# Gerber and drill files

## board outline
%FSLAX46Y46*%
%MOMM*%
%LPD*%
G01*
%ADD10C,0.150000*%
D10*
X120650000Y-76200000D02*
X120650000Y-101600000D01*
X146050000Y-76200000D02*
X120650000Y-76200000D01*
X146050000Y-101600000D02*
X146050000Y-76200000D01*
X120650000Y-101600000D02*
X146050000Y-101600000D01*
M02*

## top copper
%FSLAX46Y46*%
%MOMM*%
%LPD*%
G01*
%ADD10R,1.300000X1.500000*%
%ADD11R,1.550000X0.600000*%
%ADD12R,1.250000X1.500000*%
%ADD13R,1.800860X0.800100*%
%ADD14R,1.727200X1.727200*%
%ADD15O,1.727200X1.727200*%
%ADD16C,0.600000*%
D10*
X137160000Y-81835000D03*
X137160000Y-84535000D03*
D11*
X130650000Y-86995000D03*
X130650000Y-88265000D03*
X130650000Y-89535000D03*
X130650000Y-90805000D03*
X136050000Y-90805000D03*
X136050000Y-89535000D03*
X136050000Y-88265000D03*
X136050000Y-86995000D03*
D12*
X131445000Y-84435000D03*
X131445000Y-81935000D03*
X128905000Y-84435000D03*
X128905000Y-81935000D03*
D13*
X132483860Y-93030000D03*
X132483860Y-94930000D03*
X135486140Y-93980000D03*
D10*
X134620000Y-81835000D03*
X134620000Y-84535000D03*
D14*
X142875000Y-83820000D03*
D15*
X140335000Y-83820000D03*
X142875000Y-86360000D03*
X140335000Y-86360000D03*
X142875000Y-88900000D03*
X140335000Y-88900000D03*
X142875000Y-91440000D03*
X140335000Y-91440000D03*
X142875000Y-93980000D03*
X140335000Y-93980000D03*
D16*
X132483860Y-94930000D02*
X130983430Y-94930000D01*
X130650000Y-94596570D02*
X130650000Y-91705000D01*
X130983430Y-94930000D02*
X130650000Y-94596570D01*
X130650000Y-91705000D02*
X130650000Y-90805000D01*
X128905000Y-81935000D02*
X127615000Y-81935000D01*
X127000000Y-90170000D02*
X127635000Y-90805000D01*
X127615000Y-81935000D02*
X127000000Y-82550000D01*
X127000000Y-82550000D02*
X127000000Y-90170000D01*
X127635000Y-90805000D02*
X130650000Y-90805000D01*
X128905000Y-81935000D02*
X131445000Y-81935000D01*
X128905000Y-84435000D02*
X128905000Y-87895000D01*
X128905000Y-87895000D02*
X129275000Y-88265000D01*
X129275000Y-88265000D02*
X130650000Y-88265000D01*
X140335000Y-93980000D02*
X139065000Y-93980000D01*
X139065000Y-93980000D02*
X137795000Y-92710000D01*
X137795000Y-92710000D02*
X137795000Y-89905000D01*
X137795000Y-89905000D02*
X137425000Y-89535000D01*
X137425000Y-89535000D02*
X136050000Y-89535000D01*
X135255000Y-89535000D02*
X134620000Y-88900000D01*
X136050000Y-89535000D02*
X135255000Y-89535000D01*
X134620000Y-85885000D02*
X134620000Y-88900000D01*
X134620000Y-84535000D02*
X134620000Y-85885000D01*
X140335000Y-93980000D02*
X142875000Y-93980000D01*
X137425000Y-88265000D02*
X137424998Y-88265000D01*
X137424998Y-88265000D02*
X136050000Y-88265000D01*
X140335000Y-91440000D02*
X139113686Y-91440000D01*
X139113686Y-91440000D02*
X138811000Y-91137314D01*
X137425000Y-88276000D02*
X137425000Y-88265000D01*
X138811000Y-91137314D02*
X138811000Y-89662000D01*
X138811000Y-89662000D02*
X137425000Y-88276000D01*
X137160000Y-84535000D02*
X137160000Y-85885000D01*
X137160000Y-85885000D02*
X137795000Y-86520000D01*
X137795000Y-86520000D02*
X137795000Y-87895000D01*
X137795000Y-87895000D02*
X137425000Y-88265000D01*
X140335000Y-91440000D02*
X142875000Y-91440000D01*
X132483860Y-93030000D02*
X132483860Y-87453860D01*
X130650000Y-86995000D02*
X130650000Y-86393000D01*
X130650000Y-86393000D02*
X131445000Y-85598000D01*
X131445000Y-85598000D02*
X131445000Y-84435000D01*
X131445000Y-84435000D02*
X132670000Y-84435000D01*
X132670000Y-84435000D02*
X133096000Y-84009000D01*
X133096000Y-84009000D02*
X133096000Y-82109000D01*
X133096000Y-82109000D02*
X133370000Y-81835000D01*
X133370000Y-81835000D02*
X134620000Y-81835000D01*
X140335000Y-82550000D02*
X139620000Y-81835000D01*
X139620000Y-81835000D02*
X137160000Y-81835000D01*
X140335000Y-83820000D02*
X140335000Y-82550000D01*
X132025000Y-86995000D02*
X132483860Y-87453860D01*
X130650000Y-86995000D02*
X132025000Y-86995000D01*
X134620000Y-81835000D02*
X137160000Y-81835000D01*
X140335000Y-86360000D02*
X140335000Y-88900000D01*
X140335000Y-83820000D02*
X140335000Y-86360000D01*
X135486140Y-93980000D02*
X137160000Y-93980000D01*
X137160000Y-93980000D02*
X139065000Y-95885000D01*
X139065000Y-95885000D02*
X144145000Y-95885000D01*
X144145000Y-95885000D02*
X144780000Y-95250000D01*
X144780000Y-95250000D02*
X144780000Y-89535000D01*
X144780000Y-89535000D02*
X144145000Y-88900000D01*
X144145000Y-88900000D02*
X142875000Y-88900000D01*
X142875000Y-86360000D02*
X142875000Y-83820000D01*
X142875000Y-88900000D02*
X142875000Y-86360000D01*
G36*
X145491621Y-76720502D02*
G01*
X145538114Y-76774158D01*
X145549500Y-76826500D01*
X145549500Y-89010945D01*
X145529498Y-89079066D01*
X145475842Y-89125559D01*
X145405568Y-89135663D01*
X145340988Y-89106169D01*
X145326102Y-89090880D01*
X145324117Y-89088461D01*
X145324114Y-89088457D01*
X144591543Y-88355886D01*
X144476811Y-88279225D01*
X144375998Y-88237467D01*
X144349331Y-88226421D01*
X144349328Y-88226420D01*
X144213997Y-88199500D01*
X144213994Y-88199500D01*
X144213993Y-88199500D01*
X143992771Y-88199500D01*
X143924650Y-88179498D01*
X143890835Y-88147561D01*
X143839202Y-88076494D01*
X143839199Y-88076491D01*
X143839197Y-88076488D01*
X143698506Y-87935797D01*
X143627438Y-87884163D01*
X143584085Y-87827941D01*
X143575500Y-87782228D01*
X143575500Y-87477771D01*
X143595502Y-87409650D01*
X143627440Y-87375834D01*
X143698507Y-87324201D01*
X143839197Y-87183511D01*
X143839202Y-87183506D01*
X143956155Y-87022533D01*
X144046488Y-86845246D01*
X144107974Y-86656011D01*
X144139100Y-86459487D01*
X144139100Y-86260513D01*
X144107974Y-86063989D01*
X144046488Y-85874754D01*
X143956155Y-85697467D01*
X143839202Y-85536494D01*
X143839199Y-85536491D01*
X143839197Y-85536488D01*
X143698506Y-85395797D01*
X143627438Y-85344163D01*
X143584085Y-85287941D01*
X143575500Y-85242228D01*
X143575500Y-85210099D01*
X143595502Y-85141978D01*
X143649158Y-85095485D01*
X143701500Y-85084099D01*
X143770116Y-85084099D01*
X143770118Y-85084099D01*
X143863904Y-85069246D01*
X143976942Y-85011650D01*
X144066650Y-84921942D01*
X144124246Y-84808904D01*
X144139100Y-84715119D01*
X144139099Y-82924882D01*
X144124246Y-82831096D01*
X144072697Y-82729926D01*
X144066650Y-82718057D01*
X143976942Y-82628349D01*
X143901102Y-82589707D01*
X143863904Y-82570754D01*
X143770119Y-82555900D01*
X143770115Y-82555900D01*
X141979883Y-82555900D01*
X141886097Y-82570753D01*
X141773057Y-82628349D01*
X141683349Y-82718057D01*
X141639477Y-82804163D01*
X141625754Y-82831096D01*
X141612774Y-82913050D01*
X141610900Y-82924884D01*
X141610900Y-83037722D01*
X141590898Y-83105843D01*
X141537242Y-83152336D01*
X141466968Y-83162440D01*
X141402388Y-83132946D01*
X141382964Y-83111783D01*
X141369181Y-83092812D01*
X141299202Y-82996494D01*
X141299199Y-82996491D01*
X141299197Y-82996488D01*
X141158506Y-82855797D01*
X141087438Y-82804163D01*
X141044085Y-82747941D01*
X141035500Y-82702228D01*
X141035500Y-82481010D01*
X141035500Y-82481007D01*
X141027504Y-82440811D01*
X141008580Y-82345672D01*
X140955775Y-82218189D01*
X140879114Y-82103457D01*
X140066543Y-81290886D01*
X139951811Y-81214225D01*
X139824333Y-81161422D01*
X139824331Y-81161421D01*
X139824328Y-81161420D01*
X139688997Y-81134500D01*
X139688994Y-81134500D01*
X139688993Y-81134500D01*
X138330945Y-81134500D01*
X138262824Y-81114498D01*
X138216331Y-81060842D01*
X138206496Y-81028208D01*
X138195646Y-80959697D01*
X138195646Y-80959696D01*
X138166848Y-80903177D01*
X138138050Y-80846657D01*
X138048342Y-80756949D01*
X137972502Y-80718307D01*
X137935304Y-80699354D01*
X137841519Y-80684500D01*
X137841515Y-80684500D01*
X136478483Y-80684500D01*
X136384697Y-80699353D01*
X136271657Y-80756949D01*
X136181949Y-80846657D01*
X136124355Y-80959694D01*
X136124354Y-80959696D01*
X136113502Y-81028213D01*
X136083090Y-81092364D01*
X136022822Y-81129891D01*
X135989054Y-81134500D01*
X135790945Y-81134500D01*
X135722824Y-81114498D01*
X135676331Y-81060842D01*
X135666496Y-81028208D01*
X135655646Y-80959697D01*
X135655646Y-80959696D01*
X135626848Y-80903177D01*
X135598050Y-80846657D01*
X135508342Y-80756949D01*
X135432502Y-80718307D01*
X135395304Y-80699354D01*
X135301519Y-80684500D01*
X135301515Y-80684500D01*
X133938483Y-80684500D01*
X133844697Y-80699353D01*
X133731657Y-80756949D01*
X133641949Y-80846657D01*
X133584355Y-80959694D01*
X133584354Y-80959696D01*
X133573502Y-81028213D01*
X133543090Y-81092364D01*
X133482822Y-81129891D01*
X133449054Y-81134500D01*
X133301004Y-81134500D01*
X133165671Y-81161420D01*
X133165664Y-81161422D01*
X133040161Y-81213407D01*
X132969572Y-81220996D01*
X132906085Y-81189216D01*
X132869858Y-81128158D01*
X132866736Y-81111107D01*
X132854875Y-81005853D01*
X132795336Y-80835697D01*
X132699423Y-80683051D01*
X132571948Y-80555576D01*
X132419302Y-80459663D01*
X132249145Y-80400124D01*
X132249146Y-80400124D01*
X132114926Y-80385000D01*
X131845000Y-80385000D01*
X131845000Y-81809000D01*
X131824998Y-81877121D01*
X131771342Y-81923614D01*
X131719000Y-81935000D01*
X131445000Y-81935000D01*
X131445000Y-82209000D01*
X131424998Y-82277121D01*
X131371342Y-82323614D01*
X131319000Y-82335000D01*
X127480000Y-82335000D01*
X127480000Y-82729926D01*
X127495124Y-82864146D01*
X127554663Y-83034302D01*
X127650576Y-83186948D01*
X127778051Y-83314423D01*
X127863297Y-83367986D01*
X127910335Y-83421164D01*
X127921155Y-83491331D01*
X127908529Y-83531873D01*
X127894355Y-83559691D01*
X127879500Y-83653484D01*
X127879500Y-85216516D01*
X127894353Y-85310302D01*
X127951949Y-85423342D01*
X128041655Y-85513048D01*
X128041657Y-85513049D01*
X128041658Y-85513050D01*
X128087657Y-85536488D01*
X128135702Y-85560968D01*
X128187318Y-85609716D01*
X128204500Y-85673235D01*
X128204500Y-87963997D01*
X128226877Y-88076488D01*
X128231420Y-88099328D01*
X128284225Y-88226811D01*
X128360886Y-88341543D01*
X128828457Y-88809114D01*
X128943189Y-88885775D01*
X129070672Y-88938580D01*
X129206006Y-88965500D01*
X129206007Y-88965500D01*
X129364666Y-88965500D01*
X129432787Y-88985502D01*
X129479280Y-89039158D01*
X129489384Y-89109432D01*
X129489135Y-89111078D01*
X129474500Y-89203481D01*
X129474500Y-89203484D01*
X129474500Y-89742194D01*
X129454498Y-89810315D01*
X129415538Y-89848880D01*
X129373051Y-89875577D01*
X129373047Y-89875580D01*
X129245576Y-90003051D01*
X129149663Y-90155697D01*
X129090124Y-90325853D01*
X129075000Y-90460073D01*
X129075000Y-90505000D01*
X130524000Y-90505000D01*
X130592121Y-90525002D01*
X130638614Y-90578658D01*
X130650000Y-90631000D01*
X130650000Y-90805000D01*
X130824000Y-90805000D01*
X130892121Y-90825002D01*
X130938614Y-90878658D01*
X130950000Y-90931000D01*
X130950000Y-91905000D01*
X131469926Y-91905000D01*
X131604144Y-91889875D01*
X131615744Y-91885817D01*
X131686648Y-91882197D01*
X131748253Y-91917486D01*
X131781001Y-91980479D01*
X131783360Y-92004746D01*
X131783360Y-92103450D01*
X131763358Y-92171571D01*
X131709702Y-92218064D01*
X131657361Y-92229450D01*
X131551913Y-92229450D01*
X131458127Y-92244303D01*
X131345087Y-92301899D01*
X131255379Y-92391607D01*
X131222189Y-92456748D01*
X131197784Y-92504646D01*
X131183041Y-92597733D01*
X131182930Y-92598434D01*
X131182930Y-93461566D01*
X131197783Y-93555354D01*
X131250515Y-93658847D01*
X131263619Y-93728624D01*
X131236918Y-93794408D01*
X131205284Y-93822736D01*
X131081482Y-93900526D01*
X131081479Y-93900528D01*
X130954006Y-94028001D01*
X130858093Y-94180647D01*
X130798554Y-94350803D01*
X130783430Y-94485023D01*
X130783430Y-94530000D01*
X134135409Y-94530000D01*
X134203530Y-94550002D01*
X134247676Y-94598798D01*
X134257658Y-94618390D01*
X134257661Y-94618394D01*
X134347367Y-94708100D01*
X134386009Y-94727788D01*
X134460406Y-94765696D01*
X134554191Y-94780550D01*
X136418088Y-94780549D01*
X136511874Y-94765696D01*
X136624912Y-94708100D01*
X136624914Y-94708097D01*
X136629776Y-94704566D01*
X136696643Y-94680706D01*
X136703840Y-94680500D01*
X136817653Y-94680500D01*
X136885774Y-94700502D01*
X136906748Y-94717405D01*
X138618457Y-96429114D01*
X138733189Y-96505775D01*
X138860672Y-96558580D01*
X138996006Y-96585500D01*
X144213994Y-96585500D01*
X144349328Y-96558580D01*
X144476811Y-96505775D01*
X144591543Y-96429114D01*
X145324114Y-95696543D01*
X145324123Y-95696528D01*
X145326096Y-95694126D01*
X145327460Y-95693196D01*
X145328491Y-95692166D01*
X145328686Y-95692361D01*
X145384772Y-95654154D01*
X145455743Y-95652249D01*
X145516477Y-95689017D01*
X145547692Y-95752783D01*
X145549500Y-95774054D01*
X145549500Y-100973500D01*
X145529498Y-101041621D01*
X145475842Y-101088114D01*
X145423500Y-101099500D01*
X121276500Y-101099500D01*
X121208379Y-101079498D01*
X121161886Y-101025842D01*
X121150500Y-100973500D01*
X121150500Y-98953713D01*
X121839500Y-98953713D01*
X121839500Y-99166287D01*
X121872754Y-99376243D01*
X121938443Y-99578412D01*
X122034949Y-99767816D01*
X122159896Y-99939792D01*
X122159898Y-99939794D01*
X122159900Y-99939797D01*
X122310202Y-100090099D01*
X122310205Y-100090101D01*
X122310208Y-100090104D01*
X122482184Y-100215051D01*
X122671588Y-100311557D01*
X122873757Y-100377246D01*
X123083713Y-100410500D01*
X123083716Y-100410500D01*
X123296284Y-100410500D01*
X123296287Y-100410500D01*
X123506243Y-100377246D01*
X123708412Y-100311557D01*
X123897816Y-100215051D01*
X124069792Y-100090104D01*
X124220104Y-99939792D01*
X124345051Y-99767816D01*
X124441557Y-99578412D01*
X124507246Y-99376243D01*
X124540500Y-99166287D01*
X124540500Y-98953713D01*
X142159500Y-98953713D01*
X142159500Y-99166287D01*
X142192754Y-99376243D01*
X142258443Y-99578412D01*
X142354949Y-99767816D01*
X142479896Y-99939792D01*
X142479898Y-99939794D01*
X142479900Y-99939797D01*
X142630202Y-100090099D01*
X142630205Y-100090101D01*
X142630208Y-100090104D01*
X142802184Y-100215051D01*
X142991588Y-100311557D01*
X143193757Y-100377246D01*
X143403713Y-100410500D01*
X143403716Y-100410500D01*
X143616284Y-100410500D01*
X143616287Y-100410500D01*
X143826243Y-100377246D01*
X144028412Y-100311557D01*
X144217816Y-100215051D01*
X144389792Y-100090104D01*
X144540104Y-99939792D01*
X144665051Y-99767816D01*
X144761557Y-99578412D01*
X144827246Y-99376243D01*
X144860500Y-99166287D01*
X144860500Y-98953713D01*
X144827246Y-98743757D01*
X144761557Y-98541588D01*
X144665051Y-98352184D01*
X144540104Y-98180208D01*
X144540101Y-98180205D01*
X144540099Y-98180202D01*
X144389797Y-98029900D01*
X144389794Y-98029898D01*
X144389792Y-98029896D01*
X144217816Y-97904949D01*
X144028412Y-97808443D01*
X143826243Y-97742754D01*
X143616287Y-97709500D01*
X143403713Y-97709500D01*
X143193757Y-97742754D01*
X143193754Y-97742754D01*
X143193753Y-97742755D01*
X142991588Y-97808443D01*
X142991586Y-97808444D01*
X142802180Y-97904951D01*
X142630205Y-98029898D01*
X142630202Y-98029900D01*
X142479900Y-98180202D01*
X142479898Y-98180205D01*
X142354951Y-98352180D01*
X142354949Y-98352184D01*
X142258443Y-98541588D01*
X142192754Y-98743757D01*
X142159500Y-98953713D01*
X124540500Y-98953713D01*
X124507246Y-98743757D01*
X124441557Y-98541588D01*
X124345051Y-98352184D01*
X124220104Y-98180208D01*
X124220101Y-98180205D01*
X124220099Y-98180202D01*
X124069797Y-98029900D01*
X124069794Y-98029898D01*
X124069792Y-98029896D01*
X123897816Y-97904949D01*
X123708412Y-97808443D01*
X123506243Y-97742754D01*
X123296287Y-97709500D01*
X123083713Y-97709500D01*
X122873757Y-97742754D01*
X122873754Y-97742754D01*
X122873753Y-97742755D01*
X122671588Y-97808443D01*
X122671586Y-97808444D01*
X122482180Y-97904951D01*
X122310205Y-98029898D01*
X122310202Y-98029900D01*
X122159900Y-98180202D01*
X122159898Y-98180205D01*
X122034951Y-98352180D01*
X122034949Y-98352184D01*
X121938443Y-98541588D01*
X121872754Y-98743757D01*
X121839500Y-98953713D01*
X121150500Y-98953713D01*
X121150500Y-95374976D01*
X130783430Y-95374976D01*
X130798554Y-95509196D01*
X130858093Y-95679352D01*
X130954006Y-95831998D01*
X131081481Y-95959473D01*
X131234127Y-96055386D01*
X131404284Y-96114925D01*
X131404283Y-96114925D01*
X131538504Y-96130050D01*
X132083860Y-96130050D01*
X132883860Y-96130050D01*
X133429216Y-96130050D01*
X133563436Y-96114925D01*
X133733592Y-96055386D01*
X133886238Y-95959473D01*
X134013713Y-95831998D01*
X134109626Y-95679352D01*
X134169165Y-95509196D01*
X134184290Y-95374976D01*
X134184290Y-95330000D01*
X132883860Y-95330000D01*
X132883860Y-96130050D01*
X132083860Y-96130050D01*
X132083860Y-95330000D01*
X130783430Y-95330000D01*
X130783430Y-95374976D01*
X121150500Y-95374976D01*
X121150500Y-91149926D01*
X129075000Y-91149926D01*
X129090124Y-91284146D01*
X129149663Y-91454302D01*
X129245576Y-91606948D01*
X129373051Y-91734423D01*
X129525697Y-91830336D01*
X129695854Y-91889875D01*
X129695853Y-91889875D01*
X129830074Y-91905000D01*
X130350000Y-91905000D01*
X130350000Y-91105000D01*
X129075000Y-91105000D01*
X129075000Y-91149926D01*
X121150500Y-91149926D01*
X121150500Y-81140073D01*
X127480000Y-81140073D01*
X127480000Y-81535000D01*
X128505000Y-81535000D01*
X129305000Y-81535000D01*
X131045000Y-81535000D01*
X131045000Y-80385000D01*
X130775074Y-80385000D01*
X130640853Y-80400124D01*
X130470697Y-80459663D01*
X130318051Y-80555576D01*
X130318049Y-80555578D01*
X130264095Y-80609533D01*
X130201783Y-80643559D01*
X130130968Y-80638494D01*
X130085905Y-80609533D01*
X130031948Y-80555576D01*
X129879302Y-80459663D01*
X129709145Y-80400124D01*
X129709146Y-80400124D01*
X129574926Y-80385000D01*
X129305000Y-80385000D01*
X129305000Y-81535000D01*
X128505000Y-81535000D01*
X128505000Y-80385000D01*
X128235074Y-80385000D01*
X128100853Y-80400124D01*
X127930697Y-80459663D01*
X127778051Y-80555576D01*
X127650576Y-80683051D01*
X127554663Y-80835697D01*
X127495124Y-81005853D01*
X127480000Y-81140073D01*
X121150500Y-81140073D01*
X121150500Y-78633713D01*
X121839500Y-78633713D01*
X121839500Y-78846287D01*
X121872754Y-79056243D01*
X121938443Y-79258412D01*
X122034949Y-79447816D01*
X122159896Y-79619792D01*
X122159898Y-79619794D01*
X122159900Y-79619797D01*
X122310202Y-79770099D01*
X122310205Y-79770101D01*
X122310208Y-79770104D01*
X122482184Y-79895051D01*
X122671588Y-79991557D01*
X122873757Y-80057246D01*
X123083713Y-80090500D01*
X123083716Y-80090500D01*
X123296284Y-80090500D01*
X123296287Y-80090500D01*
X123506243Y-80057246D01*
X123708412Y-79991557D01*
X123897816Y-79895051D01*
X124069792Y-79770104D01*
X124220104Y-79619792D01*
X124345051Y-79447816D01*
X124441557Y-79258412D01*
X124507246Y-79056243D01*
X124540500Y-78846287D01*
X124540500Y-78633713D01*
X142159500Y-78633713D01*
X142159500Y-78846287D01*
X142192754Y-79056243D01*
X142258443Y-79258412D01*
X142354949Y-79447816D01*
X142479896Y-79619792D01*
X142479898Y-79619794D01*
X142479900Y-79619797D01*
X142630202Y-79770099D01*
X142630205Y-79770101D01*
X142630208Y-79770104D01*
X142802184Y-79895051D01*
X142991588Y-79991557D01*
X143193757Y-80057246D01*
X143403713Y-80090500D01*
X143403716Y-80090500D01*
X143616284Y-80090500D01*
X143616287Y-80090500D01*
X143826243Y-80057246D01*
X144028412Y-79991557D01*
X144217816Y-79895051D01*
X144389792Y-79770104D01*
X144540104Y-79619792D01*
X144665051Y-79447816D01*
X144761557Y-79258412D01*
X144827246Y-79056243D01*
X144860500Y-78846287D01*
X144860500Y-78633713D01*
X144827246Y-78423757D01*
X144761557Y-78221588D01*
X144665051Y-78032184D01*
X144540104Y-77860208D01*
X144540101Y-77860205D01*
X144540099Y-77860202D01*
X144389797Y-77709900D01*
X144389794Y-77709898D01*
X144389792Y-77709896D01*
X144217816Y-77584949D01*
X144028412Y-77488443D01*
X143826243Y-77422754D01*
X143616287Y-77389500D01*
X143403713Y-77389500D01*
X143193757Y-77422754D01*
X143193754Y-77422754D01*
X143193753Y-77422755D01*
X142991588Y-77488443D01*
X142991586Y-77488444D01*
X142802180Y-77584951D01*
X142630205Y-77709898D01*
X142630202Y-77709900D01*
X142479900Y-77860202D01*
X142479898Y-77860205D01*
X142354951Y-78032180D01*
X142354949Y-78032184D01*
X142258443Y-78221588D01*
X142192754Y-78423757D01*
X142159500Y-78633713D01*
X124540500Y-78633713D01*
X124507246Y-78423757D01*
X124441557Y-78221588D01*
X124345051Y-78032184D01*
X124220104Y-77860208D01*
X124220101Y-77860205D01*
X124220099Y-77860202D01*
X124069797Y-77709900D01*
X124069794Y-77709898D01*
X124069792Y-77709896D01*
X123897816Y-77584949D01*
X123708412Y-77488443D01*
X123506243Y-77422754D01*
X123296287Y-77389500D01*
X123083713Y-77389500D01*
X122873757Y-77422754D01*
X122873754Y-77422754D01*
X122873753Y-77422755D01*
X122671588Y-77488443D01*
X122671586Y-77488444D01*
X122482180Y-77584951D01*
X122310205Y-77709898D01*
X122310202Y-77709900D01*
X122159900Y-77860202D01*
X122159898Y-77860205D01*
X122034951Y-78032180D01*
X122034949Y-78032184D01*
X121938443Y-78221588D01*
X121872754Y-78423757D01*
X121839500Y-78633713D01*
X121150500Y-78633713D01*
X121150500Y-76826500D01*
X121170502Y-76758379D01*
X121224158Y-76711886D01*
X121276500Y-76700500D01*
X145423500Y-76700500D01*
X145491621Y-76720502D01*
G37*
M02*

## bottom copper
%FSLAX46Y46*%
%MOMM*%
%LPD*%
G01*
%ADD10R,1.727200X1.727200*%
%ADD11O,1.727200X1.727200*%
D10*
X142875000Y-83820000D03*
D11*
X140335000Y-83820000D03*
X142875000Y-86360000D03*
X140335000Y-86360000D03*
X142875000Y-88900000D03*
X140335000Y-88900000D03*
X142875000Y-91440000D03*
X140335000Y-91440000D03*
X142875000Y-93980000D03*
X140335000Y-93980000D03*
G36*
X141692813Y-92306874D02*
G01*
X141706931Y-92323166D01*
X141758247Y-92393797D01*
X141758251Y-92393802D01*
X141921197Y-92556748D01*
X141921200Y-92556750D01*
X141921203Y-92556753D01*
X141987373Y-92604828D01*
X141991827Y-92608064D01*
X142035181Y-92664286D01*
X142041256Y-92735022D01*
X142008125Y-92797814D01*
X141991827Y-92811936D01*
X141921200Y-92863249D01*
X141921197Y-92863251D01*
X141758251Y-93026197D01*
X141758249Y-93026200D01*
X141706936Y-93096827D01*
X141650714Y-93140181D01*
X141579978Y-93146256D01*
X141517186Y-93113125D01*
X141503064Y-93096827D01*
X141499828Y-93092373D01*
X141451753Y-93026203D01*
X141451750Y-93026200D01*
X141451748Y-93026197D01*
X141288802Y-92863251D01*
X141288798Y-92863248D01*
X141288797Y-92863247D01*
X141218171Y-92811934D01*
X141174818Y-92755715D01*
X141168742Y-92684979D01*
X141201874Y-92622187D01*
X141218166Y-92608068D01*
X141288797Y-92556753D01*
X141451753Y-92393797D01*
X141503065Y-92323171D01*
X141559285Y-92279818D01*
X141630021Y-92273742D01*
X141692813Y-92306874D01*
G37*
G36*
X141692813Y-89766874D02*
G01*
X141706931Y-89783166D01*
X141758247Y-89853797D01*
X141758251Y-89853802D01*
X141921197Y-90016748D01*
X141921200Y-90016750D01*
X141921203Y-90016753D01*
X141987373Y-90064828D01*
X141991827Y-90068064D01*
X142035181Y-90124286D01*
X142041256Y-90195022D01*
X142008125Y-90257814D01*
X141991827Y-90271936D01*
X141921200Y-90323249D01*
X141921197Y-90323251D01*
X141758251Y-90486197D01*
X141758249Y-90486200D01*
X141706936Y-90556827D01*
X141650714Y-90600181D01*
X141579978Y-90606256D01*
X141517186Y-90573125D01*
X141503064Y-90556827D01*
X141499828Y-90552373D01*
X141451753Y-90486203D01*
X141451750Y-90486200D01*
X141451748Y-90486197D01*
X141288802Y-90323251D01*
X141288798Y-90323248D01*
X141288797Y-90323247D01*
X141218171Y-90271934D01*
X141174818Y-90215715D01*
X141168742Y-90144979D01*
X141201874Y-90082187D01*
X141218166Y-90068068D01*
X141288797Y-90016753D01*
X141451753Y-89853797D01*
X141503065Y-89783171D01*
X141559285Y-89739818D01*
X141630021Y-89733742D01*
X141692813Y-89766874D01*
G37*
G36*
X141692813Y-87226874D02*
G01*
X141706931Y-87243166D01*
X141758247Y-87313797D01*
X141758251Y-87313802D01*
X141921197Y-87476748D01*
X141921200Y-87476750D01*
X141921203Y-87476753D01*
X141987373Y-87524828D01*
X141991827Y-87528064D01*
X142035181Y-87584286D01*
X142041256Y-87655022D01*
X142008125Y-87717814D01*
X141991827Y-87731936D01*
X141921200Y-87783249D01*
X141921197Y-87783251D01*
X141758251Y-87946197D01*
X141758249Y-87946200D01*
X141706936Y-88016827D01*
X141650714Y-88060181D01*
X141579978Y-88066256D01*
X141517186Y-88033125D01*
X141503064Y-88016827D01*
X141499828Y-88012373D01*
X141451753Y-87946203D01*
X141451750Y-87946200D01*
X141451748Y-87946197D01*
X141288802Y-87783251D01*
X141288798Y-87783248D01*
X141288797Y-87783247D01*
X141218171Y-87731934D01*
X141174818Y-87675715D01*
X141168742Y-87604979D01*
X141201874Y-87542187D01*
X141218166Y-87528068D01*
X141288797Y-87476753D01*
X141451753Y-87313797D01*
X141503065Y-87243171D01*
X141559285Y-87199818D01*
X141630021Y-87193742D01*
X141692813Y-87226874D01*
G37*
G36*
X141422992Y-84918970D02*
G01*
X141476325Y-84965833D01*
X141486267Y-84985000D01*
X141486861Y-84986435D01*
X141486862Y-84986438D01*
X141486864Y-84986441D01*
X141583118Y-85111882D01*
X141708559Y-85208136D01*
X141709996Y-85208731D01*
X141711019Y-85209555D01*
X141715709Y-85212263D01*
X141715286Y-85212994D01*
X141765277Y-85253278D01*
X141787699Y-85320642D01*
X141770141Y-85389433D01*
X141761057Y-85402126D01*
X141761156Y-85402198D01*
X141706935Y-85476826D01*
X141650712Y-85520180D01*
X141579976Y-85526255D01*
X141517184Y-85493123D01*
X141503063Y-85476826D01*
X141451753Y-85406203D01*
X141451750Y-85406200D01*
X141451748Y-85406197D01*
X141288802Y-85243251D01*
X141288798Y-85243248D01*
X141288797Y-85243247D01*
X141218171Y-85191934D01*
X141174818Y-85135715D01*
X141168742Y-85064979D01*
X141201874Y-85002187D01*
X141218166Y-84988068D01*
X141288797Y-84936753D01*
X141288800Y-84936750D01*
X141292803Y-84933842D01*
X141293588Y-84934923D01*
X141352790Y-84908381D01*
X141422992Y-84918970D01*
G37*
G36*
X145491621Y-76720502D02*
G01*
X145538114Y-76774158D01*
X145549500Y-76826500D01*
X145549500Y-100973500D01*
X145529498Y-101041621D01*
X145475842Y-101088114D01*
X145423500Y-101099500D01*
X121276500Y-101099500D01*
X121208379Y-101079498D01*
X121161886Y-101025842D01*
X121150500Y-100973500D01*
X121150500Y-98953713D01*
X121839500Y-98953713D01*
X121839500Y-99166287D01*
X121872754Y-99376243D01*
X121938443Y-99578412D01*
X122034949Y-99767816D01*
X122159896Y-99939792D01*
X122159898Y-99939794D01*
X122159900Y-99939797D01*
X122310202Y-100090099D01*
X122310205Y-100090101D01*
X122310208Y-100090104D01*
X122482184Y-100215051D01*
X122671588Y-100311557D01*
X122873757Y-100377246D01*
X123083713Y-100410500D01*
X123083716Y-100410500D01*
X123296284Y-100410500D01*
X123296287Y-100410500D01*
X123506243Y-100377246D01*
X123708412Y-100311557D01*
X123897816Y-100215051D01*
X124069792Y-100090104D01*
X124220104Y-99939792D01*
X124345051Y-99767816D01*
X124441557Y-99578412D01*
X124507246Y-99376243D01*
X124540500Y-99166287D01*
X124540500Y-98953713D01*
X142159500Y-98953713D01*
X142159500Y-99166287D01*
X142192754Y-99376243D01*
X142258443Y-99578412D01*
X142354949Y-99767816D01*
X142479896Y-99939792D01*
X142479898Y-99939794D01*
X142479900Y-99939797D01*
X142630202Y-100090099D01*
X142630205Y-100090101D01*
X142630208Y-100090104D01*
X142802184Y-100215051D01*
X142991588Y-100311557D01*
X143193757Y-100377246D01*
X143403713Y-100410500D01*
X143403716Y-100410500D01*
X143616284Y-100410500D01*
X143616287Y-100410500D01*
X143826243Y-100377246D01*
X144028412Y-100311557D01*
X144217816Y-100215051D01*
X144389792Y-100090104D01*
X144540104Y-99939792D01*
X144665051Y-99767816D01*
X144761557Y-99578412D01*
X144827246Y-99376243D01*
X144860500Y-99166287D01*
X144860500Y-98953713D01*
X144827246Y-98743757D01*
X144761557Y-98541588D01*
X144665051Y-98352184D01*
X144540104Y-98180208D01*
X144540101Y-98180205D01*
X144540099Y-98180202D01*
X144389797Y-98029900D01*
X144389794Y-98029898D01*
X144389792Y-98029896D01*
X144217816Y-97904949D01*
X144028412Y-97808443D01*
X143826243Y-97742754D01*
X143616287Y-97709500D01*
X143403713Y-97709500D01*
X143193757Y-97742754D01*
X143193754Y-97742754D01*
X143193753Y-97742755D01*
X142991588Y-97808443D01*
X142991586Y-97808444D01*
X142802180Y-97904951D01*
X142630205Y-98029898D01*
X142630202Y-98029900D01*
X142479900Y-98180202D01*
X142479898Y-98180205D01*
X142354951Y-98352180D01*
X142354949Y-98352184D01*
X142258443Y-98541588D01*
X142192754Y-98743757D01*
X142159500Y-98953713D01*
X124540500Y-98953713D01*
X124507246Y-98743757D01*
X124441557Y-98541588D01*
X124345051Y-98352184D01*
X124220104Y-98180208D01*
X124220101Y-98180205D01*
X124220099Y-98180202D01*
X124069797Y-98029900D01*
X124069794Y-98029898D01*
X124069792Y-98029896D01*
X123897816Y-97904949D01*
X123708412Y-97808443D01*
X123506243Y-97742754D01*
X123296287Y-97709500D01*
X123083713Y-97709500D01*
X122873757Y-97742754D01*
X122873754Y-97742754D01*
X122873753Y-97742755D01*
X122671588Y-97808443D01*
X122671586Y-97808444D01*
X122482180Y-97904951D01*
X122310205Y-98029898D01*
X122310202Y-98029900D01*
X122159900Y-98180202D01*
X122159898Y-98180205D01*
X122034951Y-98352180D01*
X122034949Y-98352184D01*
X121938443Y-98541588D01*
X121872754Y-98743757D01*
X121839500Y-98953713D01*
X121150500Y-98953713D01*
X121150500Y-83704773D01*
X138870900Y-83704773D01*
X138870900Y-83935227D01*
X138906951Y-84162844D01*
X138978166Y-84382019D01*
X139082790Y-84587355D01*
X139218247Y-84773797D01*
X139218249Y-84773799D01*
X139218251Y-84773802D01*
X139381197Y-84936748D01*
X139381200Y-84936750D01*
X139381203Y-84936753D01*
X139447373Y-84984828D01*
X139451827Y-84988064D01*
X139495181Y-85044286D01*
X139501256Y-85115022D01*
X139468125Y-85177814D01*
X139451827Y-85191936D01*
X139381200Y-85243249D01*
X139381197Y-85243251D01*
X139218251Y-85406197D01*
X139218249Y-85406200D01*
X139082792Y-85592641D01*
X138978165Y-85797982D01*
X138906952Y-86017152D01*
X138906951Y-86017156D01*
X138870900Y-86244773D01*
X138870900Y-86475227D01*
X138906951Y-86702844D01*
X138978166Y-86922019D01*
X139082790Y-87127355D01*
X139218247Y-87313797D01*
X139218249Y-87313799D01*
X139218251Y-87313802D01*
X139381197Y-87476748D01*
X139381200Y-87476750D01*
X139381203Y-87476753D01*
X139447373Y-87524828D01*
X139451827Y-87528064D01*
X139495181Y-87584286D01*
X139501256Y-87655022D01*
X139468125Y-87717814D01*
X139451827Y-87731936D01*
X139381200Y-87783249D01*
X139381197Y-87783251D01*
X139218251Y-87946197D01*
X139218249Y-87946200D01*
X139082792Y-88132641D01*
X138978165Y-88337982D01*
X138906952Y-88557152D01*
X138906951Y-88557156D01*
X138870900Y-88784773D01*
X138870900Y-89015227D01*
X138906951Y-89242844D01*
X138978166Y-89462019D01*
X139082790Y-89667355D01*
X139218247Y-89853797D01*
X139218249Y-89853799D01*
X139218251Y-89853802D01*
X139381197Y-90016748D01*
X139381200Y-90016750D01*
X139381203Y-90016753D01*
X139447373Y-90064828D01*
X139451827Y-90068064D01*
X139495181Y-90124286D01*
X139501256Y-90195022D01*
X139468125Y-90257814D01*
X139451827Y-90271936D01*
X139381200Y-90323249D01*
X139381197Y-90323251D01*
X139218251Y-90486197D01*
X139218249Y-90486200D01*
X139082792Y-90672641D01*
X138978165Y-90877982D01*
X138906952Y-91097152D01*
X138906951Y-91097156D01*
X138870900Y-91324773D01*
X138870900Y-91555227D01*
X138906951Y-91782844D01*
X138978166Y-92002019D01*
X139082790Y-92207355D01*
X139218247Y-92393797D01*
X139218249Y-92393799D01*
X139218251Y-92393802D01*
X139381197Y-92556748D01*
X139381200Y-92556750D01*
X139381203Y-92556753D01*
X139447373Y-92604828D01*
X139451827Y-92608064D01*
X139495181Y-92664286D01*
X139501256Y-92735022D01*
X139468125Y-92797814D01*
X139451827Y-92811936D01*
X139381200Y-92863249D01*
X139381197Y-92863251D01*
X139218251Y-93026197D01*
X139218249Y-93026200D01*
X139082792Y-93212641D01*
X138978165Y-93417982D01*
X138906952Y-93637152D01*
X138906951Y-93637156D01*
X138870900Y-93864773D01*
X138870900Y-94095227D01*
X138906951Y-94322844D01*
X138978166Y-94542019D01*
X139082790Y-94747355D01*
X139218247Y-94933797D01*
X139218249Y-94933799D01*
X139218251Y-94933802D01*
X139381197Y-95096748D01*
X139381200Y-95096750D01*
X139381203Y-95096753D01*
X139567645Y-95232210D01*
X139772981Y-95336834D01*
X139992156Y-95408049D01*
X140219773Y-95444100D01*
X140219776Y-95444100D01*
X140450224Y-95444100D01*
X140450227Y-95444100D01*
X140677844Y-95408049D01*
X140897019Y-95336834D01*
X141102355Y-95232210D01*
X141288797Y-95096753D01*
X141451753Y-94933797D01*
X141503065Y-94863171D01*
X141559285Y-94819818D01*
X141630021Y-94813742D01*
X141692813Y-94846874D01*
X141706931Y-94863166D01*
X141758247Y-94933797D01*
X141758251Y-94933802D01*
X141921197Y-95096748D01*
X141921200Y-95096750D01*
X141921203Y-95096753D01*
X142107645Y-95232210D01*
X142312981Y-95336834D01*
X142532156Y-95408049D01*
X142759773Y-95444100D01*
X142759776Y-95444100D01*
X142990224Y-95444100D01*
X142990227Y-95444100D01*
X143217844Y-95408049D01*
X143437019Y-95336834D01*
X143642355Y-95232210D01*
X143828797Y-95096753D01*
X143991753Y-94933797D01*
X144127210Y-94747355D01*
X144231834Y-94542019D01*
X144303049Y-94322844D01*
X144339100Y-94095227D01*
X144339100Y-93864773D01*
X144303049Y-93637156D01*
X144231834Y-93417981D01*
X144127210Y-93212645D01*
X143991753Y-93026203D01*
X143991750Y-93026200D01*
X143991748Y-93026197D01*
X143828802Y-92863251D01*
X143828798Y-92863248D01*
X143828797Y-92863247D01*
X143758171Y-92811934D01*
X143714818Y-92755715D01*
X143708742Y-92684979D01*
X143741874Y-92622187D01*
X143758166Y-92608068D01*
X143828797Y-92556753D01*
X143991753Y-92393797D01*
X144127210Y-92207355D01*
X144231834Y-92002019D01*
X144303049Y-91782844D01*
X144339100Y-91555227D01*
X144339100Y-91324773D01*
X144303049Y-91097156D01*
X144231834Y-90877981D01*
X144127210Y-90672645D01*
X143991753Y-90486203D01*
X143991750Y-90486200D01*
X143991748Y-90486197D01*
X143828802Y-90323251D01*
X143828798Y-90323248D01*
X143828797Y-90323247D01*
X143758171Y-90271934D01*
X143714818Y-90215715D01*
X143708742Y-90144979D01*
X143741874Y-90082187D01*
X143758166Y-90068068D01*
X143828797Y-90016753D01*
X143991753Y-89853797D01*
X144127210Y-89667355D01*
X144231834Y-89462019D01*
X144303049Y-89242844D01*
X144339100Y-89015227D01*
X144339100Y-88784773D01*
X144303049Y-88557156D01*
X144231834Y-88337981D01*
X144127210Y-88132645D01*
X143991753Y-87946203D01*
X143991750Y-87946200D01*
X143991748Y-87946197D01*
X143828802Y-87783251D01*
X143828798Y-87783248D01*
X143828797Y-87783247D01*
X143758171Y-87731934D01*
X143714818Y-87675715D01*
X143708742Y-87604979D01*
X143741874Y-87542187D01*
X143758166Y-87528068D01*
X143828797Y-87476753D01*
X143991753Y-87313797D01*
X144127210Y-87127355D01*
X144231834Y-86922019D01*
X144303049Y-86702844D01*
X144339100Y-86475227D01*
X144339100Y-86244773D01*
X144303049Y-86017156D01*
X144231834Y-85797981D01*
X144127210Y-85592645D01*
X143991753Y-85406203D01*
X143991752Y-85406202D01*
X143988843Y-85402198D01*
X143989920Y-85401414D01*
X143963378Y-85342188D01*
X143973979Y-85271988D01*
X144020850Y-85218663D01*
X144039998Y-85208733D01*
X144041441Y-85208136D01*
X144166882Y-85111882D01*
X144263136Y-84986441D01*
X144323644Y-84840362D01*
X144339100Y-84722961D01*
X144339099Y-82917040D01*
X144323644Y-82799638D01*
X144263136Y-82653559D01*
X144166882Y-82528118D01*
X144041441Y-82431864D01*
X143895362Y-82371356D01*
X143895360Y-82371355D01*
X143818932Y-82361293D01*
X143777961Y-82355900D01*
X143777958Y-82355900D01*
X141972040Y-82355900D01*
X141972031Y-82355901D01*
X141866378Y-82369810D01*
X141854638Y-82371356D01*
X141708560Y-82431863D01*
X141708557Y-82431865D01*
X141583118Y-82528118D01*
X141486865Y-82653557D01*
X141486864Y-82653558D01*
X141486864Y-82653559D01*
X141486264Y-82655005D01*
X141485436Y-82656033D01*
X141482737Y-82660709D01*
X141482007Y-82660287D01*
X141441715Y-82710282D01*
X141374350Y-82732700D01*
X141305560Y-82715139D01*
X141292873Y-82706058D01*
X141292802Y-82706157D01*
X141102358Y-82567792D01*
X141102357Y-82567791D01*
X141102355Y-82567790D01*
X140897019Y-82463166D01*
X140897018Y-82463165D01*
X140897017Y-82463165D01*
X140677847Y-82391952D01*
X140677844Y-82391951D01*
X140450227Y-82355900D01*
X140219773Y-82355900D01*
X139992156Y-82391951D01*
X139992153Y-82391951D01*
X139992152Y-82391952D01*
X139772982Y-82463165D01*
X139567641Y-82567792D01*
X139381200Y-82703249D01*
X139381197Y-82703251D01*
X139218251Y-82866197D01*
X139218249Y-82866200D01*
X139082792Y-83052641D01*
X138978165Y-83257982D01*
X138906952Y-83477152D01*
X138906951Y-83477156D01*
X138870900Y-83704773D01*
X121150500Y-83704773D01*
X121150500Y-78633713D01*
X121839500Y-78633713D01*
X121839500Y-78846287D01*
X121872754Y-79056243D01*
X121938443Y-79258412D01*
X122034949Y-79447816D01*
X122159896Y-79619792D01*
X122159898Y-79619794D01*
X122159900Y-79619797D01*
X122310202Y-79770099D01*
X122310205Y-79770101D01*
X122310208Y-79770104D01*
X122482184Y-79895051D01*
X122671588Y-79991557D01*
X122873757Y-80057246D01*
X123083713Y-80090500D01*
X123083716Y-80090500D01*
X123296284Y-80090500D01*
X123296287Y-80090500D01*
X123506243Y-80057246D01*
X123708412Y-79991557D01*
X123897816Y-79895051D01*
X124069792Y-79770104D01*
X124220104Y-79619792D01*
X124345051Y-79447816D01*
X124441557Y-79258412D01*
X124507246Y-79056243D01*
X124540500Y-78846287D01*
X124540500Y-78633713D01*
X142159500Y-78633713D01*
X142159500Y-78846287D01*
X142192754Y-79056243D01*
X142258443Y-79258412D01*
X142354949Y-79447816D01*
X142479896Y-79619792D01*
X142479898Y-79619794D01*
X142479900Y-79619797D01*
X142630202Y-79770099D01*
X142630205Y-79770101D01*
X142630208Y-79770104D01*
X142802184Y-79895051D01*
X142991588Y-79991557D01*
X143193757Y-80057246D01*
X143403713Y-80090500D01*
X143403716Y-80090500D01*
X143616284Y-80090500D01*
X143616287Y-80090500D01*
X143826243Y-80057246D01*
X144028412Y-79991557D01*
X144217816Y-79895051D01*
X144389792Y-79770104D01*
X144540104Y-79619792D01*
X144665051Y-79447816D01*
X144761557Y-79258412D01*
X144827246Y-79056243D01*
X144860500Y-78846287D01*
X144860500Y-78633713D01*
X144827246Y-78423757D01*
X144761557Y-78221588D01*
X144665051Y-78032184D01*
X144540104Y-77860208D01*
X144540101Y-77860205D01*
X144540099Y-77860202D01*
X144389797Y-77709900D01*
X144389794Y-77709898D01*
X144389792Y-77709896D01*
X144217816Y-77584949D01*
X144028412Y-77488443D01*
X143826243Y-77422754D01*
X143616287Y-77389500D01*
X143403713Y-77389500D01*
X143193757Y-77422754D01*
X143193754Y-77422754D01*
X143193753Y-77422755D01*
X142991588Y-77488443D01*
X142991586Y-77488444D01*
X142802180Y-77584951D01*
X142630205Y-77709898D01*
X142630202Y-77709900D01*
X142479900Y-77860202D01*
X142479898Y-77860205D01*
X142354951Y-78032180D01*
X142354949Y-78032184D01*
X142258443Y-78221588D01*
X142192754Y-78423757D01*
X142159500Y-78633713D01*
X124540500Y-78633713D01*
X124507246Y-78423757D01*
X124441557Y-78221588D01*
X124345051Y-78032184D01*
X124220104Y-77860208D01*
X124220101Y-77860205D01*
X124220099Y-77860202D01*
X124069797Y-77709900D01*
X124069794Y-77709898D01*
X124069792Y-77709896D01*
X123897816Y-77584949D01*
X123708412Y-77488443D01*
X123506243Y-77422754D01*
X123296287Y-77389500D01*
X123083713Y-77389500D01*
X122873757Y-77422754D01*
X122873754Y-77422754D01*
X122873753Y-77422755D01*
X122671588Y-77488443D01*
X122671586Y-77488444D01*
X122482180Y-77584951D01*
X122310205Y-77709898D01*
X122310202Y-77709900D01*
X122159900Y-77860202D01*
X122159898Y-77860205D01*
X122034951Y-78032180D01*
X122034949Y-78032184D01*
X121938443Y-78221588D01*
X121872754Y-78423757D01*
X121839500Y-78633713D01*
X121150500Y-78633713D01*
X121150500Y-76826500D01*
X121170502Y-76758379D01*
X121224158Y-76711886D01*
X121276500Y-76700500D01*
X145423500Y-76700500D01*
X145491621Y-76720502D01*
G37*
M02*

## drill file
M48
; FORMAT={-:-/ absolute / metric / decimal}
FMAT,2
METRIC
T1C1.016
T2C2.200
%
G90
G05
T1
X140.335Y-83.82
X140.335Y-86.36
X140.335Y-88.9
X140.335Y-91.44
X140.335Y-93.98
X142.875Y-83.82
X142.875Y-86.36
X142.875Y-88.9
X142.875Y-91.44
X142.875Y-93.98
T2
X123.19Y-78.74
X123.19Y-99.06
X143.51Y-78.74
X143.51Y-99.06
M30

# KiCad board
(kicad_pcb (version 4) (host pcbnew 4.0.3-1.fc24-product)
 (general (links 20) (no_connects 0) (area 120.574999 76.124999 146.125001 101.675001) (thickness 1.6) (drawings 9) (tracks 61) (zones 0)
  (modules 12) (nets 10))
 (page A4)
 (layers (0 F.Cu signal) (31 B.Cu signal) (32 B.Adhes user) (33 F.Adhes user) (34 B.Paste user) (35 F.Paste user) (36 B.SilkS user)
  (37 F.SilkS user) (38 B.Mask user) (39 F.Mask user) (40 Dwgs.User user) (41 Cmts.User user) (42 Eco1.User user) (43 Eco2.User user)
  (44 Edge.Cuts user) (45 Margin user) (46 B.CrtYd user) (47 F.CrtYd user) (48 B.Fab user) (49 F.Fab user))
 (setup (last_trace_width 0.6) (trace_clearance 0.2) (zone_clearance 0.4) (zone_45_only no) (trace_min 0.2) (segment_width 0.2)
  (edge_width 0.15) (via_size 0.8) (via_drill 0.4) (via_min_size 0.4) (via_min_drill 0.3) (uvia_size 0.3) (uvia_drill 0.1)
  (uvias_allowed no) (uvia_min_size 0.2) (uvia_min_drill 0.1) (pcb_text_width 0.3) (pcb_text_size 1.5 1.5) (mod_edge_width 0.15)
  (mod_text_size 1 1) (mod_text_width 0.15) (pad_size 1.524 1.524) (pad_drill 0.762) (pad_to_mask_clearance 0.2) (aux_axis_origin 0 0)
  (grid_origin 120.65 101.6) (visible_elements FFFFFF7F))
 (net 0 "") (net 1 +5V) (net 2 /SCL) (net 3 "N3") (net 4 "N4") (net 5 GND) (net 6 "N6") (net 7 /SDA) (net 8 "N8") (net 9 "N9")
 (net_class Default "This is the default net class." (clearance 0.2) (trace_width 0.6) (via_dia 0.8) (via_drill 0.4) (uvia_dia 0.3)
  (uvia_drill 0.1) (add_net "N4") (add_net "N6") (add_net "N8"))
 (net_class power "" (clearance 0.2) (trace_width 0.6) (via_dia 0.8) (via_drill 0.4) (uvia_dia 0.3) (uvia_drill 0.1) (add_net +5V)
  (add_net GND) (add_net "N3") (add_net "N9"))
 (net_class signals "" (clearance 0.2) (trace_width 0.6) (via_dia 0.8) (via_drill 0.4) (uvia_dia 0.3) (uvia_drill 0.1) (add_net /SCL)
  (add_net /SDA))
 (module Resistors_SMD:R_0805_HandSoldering (layer F.Cu) (at 137.16 83.185 270)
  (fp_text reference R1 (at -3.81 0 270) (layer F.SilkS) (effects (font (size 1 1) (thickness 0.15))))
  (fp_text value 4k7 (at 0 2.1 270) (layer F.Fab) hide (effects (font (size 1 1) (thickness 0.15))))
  (pad 1 smd rect (at -1.35 0 270) (size 1.5 1.3) (layers F.Cu F.Paste F.Mask) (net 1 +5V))
  (pad 2 smd rect (at 1.35 0 270) (size 1.5 1.3) (layers F.Cu F.Paste F.Mask) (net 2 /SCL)))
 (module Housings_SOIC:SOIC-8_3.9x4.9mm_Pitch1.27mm (layer F.Cu) (at 133.35 88.9)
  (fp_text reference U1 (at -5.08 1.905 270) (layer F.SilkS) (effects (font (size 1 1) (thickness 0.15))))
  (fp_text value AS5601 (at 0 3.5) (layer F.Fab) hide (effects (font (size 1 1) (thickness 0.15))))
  (pad 1 smd rect (at -2.7 -1.905) (size 1.55 0.6) (layers F.Cu F.Paste F.Mask) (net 1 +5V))
  (pad 2 smd rect (at -2.7 -0.635) (size 1.55 0.6) (layers F.Cu F.Paste F.Mask) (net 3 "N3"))
  (pad 3 smd rect (at -2.7 0.635) (size 1.55 0.6) (layers F.Cu F.Paste F.Mask) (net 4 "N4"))
  (pad 4 smd rect (at -2.7 1.905) (size 1.55 0.6) (layers F.Cu F.Paste F.Mask) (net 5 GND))
  (pad 5 smd rect (at 2.7 1.905) (size 1.55 0.6) (layers F.Cu F.Paste F.Mask) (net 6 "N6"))
  (pad 6 smd rect (at 2.7 0.635) (size 1.55 0.6) (layers F.Cu F.Paste F.Mask) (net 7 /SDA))
  (pad 7 smd rect (at 2.7 -0.635) (size 1.55 0.6) (layers F.Cu F.Paste F.Mask) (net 2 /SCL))
  (pad 8 smd rect (at 2.7 -1.905) (size 1.55 0.6) (layers F.Cu F.Paste F.Mask) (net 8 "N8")))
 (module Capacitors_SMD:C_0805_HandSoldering (layer F.Cu) (at 131.445 83.185 90)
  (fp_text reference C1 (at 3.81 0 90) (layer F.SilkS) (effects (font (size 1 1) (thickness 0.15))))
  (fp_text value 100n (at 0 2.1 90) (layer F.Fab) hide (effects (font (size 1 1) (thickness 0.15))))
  (pad 1 smd rect (at -1.25 0 90) (size 1.5 1.25) (layers F.Cu F.Paste F.Mask) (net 1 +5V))
  (pad 2 smd rect (at 1.25 0 90) (size 1.5 1.25) (layers F.Cu F.Paste F.Mask) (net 5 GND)))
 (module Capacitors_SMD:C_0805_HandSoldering (layer F.Cu) (at 128.905 83.185 90)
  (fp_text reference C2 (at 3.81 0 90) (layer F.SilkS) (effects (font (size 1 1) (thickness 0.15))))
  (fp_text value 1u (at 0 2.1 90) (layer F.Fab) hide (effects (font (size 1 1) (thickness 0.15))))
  (pad 1 smd rect (at -1.25 0 90) (size 1.5 1.25) (layers F.Cu F.Paste F.Mask) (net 3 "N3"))
  (pad 2 smd rect (at 1.25 0 90) (size 1.5 1.25) (layers F.Cu F.Paste F.Mask) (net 5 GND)))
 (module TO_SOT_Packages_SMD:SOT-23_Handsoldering (layer F.Cu) (at 133.985 93.98 270)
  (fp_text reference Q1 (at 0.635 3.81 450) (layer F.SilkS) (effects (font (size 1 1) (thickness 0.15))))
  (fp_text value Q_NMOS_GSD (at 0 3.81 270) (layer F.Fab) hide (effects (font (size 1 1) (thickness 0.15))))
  (pad 1 smd rect (at -0.95 1.50114 270) (size 0.8001 1.80086) (layers F.Cu F.Paste F.Mask) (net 1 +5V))
  (pad 2 smd rect (at 0.95 1.50114 270) (size 0.8001 1.80086) (layers F.Cu F.Paste F.Mask) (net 5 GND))
  (pad 3 smd rect (at 0 -1.50114 270) (size 0.8001 1.80086) (layers F.Cu F.Paste F.Mask) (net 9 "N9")))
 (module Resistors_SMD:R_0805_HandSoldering (layer F.Cu) (at 134.62 83.185 270)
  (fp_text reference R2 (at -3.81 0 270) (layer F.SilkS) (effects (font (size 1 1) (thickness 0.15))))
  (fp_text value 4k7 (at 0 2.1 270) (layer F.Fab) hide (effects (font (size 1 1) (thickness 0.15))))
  (pad 1 smd rect (at -1.35 0 270) (size 1.5 1.3) (layers F.Cu F.Paste F.Mask) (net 1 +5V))
  (pad 2 smd rect (at 1.35 0 270) (size 1.5 1.3) (layers F.Cu F.Paste F.Mask) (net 7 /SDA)))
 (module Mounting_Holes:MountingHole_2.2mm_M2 (layer F.Cu) (at 123.19 78.74)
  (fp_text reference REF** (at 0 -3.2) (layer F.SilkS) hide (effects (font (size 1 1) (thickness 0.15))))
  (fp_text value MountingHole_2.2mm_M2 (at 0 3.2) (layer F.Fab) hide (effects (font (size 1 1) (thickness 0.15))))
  (pad 1 np_thru_hole circle (at 0 0) (size 2.2 2.2) (drill 2.2) (layers *.Cu *.Mask F.SilkS)))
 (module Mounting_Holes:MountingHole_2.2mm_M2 (layer F.Cu) (at 123.19 99.06)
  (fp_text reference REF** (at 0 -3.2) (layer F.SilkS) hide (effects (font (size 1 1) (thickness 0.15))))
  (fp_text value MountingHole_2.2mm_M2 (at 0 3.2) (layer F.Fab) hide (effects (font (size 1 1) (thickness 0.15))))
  (pad 1 np_thru_hole circle (at 0 0) (size 2.2 2.2) (drill 2.2) (layers *.Cu *.Mask F.SilkS)))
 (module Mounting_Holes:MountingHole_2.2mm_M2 (layer F.Cu) (at 143.51 78.74)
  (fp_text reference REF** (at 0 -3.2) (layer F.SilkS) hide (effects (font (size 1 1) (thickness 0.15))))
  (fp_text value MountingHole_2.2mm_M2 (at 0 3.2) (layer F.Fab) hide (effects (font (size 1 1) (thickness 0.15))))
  (pad 1 np_thru_hole circle (at 0 0) (size 2.2 2.2) (drill 2.2) (layers *.Cu *.Mask F.SilkS)))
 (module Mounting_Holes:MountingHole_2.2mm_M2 (layer F.Cu) (at 143.51 99.06)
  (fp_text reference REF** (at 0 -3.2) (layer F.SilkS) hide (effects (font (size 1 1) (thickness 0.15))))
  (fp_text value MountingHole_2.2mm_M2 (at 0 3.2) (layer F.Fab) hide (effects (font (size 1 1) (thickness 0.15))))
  (pad 1 np_thru_hole circle (at 0 0) (size 2.2 2.2) (drill 2.2) (layers *.Cu *.Mask F.SilkS)))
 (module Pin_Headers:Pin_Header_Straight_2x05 (layer B.Cu) (at 142.875 83.82 180)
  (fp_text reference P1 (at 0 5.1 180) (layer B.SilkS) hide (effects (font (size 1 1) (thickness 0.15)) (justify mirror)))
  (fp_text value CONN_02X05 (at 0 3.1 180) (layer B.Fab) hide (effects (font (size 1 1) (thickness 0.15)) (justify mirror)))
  (pad 1 thru_hole rect (at 0 0 180) (size 1.7272 1.7272) (drill 1.016) (layers *.Cu *.Mask B.SilkS) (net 9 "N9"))
  (pad 2 thru_hole oval (at 2.54 0 180) (size 1.7272 1.7272) (drill 1.016) (layers *.Cu *.Mask B.SilkS) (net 1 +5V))
  (pad 3 thru_hole oval (at 0 -2.54 180) (size 1.7272 1.7272) (drill 1.016) (layers *.Cu *.Mask B.SilkS) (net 9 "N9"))
  (pad 4 thru_hole oval (at 2.54 -2.54 180) (size 1.7272 1.7272) (drill 1.016) (layers *.Cu *.Mask B.SilkS) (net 1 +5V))
  (pad 5 thru_hole oval (at 0 -5.08 180) (size 1.7272 1.7272) (drill 1.016) (layers *.Cu *.Mask B.SilkS) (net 9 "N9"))
  (pad 6 thru_hole oval (at 2.54 -5.08 180) (size 1.7272 1.7272) (drill 1.016) (layers *.Cu *.Mask B.SilkS) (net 1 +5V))
  (pad 7 thru_hole oval (at 0 -7.62 180) (size 1.7272 1.7272) (drill 1.016) (layers *.Cu *.Mask B.SilkS) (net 2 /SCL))
  (pad 8 thru_hole oval (at 2.54 -7.62 180) (size 1.7272 1.7272) (drill 1.016) (layers *.Cu *.Mask B.SilkS) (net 2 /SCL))
  (pad 9 thru_hole oval (at 0 -10.16 180) (size 1.7272 1.7272) (drill 1.016) (layers *.Cu *.Mask B.SilkS) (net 7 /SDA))
  (pad 10 thru_hole oval (at 2.54 -10.16 180) (size 1.7272 1.7272) (drill 1.016) (layers *.Cu *.Mask B.SilkS) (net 7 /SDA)))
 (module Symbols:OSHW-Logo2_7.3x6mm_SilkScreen (layer B.Cu) (at 128.905 92.71 180)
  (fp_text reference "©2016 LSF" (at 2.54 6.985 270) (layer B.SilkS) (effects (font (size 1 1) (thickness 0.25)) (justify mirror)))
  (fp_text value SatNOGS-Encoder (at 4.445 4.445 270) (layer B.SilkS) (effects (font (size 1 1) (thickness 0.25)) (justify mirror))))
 (gr_line (start 120.65 76.2) (end 120.65 101.6) (layer Edge.Cuts) (width 0.15))
 (gr_line (start 146.05 76.2) (end 120.65 76.2) (layer Edge.Cuts) (width 0.15))
 (gr_line (start 146.05 101.6) (end 146.05 76.2) (layer Edge.Cuts) (width 0.15))
 (gr_line (start 120.65 101.6) (end 146.05 101.6) (layer Edge.Cuts) (width 0.15))
 (segment (start 132.48386 94.93) (end 130.98343 94.93) (width 0.6) (layer F.Cu) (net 5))
 (segment (start 130.65 94.59657) (end 130.65 91.705) (width 0.6) (layer F.Cu) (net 5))
 (segment (start 130.98343 94.93) (end 130.65 94.59657) (width 0.6) (layer F.Cu) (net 5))
 (segment (start 130.65 91.705) (end 130.65 90.805) (width 0.6) (layer F.Cu) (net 5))
 (segment (start 128.905 81.935) (end 127.615 81.935) (width 0.6) (layer F.Cu) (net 5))
 (segment (start 127 90.17) (end 127.635 90.805) (width 0.6) (layer F.Cu) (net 5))
 (segment (start 127.615 81.935) (end 127 82.55) (width 0.6) (layer F.Cu) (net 5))
 (segment (start 127 82.55) (end 127 90.17) (width 0.6) (layer F.Cu) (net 5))
 (segment (start 127.635 90.805) (end 130.65 90.805) (width 0.6) (layer F.Cu) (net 5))
 (segment (start 128.905 81.935) (end 131.445 81.935) (width 0.6) (layer F.Cu) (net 5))
 (segment (start 128.905 84.435) (end 128.905 87.895) (width 0.6) (layer F.Cu) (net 3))
 (segment (start 128.905 87.895) (end 129.275 88.265) (width 0.6) (layer F.Cu) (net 3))
 (segment (start 129.275 88.265) (end 130.65 88.265) (width 0.6) (layer F.Cu) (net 3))
 (segment (start 140.335 93.98) (end 139.065 93.98) (width 0.6) (layer F.Cu) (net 7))
 (segment (start 139.065 93.98) (end 137.795 92.71) (width 0.6) (layer F.Cu) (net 7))
 (segment (start 137.795 92.71) (end 137.795 89.905) (width 0.6) (layer F.Cu) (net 7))
 (segment (start 137.795 89.905) (end 137.425 89.535) (width 0.6) (layer F.Cu) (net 7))
 (segment (start 137.425 89.535) (end 136.05 89.535) (width 0.6) (layer F.Cu) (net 7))
 (segment (start 135.255 89.535) (end 134.62 88.9) (width 0.6) (layer F.Cu) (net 7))
 (segment (start 136.05 89.535) (end 135.255 89.535) (width 0.6) (layer F.Cu) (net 7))
 (segment (start 134.62 85.885) (end 134.62 88.9) (width 0.6) (layer F.Cu) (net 7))
 (segment (start 134.62 84.535) (end 134.62 85.885) (width 0.6) (layer F.Cu) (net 7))
 (segment (start 140.335 93.98) (end 142.875 93.98) (width 0.6) (layer F.Cu) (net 7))
 (segment (start 137.425 88.265) (end 137.424998 88.265) (width 0.6) (layer F.Cu) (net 2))
 (segment (start 137.424998 88.265) (end 136.05 88.265) (width 0.6) (layer F.Cu) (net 2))
 (segment (start 140.335 91.44) (end 139.113686 91.44) (width 0.6) (layer F.Cu) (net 2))
 (segment (start 139.113686 91.44) (end 138.811 91.137314) (width 0.6) (layer F.Cu) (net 2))
 (segment (start 137.425 88.276) (end 137.425 88.265) (width 0.6) (layer F.Cu) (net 2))
 (segment (start 138.811 91.137314) (end 138.811 89.662) (width 0.6) (layer F.Cu) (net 2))
 (segment (start 138.811 89.662) (end 137.425 88.276) (width 0.6) (layer F.Cu) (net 2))
 (segment (start 137.16 84.535) (end 137.16 85.885) (width 0.6) (layer F.Cu) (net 2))
 (segment (start 137.16 85.885) (end 137.795 86.52) (width 0.6) (layer F.Cu) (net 2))
 (segment (start 137.795 86.52) (end 137.795 87.895) (width 0.6) (layer F.Cu) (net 2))
 (segment (start 137.795 87.895) (end 137.425 88.265) (width 0.6) (layer F.Cu) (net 2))
 (segment (start 140.335 91.44) (end 142.875 91.44) (width 0.6) (layer F.Cu) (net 2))
 (segment (start 132.48386 93.03) (end 132.48386 87.45386) (width 0.6) (layer F.Cu) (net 1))
 (segment (start 130.65 86.995) (end 130.65 86.393) (width 0.6) (layer F.Cu) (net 1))
 (segment (start 130.65 86.393) (end 131.445 85.598) (width 0.6) (layer F.Cu) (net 1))
 (segment (start 131.445 85.598) (end 131.445 84.435) (width 0.6) (layer F.Cu) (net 1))
 (segment (start 131.445 84.435) (end 132.67 84.435) (width 0.6) (layer F.Cu) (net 1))
 (segment (start 132.67 84.435) (end 133.096 84.009) (width 0.6) (layer F.Cu) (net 1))
 (segment (start 133.096 84.009) (end 133.096 82.109) (width 0.6) (layer F.Cu) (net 1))
 (segment (start 133.096 82.109) (end 133.37 81.835) (width 0.6) (layer F.Cu) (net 1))
 (segment (start 133.37 81.835) (end 134.62 81.835) (width 0.6) (layer F.Cu) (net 1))
 (segment (start 140.335 82.55) (end 139.62 81.835) (width 0.6) (layer F.Cu) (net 1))
 (segment (start 139.62 81.835) (end 137.16 81.835) (width 0.6) (layer F.Cu) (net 1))
 (segment (start 140.335 83.82) (end 140.335 82.55) (width 0.6) (layer F.Cu) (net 1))
 (segment (start 132.025 86.995) (end 132.48386 87.45386) (width 0.6) (layer F.Cu) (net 1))
 (segment (start 130.65 86.995) (end 132.025 86.995) (width 0.6) (layer F.Cu) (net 1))
 (segment (start 134.62 81.835) (end 137.16 81.835) (width 0.6) (layer F.Cu) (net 1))
 (segment (start 140.335 86.36) (end 140.335 88.9) (width 0.6) (layer F.Cu) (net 1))
 (segment (start 140.335 83.82) (end 140.335 86.36) (width 0.6) (layer F.Cu) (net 1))
 (segment (start 135.48614 93.98) (end 137.16 93.98) (width 0.6) (layer F.Cu) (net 9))
 (segment (start 137.16 93.98) (end 139.065 95.885) (width 0.6) (layer F.Cu) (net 9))
 (segment (start 139.065 95.885) (end 144.145 95.885) (width 0.6) (layer F.Cu) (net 9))
 (segment (start 144.145 95.885) (end 144.78 95.25) (width 0.6) (layer F.Cu) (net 9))
 (segment (start 144.78 95.25) (end 144.78 89.535) (width 0.6) (layer F.Cu) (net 9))
 (segment (start 144.78 89.535) (end 144.145 88.9) (width 0.6) (layer F.Cu) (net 9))
 (segment (start 144.145 88.9) (end 142.875 88.9) (width 0.6) (layer F.Cu) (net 9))
 (segment (start 142.875 86.36) (end 142.875 83.82) (width 0.6) (layer F.Cu) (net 9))
 (segment (start 142.875 88.9) (end 142.875 86.36) (width 0.6) (layer F.Cu) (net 9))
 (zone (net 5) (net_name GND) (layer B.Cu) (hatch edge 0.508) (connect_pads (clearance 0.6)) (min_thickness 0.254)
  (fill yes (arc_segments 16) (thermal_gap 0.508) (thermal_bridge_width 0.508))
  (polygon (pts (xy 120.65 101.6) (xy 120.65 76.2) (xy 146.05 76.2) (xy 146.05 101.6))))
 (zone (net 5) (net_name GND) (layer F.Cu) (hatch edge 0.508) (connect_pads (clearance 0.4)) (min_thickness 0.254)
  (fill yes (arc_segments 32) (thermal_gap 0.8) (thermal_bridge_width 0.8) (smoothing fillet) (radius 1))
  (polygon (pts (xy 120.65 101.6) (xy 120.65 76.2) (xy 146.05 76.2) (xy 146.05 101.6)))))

